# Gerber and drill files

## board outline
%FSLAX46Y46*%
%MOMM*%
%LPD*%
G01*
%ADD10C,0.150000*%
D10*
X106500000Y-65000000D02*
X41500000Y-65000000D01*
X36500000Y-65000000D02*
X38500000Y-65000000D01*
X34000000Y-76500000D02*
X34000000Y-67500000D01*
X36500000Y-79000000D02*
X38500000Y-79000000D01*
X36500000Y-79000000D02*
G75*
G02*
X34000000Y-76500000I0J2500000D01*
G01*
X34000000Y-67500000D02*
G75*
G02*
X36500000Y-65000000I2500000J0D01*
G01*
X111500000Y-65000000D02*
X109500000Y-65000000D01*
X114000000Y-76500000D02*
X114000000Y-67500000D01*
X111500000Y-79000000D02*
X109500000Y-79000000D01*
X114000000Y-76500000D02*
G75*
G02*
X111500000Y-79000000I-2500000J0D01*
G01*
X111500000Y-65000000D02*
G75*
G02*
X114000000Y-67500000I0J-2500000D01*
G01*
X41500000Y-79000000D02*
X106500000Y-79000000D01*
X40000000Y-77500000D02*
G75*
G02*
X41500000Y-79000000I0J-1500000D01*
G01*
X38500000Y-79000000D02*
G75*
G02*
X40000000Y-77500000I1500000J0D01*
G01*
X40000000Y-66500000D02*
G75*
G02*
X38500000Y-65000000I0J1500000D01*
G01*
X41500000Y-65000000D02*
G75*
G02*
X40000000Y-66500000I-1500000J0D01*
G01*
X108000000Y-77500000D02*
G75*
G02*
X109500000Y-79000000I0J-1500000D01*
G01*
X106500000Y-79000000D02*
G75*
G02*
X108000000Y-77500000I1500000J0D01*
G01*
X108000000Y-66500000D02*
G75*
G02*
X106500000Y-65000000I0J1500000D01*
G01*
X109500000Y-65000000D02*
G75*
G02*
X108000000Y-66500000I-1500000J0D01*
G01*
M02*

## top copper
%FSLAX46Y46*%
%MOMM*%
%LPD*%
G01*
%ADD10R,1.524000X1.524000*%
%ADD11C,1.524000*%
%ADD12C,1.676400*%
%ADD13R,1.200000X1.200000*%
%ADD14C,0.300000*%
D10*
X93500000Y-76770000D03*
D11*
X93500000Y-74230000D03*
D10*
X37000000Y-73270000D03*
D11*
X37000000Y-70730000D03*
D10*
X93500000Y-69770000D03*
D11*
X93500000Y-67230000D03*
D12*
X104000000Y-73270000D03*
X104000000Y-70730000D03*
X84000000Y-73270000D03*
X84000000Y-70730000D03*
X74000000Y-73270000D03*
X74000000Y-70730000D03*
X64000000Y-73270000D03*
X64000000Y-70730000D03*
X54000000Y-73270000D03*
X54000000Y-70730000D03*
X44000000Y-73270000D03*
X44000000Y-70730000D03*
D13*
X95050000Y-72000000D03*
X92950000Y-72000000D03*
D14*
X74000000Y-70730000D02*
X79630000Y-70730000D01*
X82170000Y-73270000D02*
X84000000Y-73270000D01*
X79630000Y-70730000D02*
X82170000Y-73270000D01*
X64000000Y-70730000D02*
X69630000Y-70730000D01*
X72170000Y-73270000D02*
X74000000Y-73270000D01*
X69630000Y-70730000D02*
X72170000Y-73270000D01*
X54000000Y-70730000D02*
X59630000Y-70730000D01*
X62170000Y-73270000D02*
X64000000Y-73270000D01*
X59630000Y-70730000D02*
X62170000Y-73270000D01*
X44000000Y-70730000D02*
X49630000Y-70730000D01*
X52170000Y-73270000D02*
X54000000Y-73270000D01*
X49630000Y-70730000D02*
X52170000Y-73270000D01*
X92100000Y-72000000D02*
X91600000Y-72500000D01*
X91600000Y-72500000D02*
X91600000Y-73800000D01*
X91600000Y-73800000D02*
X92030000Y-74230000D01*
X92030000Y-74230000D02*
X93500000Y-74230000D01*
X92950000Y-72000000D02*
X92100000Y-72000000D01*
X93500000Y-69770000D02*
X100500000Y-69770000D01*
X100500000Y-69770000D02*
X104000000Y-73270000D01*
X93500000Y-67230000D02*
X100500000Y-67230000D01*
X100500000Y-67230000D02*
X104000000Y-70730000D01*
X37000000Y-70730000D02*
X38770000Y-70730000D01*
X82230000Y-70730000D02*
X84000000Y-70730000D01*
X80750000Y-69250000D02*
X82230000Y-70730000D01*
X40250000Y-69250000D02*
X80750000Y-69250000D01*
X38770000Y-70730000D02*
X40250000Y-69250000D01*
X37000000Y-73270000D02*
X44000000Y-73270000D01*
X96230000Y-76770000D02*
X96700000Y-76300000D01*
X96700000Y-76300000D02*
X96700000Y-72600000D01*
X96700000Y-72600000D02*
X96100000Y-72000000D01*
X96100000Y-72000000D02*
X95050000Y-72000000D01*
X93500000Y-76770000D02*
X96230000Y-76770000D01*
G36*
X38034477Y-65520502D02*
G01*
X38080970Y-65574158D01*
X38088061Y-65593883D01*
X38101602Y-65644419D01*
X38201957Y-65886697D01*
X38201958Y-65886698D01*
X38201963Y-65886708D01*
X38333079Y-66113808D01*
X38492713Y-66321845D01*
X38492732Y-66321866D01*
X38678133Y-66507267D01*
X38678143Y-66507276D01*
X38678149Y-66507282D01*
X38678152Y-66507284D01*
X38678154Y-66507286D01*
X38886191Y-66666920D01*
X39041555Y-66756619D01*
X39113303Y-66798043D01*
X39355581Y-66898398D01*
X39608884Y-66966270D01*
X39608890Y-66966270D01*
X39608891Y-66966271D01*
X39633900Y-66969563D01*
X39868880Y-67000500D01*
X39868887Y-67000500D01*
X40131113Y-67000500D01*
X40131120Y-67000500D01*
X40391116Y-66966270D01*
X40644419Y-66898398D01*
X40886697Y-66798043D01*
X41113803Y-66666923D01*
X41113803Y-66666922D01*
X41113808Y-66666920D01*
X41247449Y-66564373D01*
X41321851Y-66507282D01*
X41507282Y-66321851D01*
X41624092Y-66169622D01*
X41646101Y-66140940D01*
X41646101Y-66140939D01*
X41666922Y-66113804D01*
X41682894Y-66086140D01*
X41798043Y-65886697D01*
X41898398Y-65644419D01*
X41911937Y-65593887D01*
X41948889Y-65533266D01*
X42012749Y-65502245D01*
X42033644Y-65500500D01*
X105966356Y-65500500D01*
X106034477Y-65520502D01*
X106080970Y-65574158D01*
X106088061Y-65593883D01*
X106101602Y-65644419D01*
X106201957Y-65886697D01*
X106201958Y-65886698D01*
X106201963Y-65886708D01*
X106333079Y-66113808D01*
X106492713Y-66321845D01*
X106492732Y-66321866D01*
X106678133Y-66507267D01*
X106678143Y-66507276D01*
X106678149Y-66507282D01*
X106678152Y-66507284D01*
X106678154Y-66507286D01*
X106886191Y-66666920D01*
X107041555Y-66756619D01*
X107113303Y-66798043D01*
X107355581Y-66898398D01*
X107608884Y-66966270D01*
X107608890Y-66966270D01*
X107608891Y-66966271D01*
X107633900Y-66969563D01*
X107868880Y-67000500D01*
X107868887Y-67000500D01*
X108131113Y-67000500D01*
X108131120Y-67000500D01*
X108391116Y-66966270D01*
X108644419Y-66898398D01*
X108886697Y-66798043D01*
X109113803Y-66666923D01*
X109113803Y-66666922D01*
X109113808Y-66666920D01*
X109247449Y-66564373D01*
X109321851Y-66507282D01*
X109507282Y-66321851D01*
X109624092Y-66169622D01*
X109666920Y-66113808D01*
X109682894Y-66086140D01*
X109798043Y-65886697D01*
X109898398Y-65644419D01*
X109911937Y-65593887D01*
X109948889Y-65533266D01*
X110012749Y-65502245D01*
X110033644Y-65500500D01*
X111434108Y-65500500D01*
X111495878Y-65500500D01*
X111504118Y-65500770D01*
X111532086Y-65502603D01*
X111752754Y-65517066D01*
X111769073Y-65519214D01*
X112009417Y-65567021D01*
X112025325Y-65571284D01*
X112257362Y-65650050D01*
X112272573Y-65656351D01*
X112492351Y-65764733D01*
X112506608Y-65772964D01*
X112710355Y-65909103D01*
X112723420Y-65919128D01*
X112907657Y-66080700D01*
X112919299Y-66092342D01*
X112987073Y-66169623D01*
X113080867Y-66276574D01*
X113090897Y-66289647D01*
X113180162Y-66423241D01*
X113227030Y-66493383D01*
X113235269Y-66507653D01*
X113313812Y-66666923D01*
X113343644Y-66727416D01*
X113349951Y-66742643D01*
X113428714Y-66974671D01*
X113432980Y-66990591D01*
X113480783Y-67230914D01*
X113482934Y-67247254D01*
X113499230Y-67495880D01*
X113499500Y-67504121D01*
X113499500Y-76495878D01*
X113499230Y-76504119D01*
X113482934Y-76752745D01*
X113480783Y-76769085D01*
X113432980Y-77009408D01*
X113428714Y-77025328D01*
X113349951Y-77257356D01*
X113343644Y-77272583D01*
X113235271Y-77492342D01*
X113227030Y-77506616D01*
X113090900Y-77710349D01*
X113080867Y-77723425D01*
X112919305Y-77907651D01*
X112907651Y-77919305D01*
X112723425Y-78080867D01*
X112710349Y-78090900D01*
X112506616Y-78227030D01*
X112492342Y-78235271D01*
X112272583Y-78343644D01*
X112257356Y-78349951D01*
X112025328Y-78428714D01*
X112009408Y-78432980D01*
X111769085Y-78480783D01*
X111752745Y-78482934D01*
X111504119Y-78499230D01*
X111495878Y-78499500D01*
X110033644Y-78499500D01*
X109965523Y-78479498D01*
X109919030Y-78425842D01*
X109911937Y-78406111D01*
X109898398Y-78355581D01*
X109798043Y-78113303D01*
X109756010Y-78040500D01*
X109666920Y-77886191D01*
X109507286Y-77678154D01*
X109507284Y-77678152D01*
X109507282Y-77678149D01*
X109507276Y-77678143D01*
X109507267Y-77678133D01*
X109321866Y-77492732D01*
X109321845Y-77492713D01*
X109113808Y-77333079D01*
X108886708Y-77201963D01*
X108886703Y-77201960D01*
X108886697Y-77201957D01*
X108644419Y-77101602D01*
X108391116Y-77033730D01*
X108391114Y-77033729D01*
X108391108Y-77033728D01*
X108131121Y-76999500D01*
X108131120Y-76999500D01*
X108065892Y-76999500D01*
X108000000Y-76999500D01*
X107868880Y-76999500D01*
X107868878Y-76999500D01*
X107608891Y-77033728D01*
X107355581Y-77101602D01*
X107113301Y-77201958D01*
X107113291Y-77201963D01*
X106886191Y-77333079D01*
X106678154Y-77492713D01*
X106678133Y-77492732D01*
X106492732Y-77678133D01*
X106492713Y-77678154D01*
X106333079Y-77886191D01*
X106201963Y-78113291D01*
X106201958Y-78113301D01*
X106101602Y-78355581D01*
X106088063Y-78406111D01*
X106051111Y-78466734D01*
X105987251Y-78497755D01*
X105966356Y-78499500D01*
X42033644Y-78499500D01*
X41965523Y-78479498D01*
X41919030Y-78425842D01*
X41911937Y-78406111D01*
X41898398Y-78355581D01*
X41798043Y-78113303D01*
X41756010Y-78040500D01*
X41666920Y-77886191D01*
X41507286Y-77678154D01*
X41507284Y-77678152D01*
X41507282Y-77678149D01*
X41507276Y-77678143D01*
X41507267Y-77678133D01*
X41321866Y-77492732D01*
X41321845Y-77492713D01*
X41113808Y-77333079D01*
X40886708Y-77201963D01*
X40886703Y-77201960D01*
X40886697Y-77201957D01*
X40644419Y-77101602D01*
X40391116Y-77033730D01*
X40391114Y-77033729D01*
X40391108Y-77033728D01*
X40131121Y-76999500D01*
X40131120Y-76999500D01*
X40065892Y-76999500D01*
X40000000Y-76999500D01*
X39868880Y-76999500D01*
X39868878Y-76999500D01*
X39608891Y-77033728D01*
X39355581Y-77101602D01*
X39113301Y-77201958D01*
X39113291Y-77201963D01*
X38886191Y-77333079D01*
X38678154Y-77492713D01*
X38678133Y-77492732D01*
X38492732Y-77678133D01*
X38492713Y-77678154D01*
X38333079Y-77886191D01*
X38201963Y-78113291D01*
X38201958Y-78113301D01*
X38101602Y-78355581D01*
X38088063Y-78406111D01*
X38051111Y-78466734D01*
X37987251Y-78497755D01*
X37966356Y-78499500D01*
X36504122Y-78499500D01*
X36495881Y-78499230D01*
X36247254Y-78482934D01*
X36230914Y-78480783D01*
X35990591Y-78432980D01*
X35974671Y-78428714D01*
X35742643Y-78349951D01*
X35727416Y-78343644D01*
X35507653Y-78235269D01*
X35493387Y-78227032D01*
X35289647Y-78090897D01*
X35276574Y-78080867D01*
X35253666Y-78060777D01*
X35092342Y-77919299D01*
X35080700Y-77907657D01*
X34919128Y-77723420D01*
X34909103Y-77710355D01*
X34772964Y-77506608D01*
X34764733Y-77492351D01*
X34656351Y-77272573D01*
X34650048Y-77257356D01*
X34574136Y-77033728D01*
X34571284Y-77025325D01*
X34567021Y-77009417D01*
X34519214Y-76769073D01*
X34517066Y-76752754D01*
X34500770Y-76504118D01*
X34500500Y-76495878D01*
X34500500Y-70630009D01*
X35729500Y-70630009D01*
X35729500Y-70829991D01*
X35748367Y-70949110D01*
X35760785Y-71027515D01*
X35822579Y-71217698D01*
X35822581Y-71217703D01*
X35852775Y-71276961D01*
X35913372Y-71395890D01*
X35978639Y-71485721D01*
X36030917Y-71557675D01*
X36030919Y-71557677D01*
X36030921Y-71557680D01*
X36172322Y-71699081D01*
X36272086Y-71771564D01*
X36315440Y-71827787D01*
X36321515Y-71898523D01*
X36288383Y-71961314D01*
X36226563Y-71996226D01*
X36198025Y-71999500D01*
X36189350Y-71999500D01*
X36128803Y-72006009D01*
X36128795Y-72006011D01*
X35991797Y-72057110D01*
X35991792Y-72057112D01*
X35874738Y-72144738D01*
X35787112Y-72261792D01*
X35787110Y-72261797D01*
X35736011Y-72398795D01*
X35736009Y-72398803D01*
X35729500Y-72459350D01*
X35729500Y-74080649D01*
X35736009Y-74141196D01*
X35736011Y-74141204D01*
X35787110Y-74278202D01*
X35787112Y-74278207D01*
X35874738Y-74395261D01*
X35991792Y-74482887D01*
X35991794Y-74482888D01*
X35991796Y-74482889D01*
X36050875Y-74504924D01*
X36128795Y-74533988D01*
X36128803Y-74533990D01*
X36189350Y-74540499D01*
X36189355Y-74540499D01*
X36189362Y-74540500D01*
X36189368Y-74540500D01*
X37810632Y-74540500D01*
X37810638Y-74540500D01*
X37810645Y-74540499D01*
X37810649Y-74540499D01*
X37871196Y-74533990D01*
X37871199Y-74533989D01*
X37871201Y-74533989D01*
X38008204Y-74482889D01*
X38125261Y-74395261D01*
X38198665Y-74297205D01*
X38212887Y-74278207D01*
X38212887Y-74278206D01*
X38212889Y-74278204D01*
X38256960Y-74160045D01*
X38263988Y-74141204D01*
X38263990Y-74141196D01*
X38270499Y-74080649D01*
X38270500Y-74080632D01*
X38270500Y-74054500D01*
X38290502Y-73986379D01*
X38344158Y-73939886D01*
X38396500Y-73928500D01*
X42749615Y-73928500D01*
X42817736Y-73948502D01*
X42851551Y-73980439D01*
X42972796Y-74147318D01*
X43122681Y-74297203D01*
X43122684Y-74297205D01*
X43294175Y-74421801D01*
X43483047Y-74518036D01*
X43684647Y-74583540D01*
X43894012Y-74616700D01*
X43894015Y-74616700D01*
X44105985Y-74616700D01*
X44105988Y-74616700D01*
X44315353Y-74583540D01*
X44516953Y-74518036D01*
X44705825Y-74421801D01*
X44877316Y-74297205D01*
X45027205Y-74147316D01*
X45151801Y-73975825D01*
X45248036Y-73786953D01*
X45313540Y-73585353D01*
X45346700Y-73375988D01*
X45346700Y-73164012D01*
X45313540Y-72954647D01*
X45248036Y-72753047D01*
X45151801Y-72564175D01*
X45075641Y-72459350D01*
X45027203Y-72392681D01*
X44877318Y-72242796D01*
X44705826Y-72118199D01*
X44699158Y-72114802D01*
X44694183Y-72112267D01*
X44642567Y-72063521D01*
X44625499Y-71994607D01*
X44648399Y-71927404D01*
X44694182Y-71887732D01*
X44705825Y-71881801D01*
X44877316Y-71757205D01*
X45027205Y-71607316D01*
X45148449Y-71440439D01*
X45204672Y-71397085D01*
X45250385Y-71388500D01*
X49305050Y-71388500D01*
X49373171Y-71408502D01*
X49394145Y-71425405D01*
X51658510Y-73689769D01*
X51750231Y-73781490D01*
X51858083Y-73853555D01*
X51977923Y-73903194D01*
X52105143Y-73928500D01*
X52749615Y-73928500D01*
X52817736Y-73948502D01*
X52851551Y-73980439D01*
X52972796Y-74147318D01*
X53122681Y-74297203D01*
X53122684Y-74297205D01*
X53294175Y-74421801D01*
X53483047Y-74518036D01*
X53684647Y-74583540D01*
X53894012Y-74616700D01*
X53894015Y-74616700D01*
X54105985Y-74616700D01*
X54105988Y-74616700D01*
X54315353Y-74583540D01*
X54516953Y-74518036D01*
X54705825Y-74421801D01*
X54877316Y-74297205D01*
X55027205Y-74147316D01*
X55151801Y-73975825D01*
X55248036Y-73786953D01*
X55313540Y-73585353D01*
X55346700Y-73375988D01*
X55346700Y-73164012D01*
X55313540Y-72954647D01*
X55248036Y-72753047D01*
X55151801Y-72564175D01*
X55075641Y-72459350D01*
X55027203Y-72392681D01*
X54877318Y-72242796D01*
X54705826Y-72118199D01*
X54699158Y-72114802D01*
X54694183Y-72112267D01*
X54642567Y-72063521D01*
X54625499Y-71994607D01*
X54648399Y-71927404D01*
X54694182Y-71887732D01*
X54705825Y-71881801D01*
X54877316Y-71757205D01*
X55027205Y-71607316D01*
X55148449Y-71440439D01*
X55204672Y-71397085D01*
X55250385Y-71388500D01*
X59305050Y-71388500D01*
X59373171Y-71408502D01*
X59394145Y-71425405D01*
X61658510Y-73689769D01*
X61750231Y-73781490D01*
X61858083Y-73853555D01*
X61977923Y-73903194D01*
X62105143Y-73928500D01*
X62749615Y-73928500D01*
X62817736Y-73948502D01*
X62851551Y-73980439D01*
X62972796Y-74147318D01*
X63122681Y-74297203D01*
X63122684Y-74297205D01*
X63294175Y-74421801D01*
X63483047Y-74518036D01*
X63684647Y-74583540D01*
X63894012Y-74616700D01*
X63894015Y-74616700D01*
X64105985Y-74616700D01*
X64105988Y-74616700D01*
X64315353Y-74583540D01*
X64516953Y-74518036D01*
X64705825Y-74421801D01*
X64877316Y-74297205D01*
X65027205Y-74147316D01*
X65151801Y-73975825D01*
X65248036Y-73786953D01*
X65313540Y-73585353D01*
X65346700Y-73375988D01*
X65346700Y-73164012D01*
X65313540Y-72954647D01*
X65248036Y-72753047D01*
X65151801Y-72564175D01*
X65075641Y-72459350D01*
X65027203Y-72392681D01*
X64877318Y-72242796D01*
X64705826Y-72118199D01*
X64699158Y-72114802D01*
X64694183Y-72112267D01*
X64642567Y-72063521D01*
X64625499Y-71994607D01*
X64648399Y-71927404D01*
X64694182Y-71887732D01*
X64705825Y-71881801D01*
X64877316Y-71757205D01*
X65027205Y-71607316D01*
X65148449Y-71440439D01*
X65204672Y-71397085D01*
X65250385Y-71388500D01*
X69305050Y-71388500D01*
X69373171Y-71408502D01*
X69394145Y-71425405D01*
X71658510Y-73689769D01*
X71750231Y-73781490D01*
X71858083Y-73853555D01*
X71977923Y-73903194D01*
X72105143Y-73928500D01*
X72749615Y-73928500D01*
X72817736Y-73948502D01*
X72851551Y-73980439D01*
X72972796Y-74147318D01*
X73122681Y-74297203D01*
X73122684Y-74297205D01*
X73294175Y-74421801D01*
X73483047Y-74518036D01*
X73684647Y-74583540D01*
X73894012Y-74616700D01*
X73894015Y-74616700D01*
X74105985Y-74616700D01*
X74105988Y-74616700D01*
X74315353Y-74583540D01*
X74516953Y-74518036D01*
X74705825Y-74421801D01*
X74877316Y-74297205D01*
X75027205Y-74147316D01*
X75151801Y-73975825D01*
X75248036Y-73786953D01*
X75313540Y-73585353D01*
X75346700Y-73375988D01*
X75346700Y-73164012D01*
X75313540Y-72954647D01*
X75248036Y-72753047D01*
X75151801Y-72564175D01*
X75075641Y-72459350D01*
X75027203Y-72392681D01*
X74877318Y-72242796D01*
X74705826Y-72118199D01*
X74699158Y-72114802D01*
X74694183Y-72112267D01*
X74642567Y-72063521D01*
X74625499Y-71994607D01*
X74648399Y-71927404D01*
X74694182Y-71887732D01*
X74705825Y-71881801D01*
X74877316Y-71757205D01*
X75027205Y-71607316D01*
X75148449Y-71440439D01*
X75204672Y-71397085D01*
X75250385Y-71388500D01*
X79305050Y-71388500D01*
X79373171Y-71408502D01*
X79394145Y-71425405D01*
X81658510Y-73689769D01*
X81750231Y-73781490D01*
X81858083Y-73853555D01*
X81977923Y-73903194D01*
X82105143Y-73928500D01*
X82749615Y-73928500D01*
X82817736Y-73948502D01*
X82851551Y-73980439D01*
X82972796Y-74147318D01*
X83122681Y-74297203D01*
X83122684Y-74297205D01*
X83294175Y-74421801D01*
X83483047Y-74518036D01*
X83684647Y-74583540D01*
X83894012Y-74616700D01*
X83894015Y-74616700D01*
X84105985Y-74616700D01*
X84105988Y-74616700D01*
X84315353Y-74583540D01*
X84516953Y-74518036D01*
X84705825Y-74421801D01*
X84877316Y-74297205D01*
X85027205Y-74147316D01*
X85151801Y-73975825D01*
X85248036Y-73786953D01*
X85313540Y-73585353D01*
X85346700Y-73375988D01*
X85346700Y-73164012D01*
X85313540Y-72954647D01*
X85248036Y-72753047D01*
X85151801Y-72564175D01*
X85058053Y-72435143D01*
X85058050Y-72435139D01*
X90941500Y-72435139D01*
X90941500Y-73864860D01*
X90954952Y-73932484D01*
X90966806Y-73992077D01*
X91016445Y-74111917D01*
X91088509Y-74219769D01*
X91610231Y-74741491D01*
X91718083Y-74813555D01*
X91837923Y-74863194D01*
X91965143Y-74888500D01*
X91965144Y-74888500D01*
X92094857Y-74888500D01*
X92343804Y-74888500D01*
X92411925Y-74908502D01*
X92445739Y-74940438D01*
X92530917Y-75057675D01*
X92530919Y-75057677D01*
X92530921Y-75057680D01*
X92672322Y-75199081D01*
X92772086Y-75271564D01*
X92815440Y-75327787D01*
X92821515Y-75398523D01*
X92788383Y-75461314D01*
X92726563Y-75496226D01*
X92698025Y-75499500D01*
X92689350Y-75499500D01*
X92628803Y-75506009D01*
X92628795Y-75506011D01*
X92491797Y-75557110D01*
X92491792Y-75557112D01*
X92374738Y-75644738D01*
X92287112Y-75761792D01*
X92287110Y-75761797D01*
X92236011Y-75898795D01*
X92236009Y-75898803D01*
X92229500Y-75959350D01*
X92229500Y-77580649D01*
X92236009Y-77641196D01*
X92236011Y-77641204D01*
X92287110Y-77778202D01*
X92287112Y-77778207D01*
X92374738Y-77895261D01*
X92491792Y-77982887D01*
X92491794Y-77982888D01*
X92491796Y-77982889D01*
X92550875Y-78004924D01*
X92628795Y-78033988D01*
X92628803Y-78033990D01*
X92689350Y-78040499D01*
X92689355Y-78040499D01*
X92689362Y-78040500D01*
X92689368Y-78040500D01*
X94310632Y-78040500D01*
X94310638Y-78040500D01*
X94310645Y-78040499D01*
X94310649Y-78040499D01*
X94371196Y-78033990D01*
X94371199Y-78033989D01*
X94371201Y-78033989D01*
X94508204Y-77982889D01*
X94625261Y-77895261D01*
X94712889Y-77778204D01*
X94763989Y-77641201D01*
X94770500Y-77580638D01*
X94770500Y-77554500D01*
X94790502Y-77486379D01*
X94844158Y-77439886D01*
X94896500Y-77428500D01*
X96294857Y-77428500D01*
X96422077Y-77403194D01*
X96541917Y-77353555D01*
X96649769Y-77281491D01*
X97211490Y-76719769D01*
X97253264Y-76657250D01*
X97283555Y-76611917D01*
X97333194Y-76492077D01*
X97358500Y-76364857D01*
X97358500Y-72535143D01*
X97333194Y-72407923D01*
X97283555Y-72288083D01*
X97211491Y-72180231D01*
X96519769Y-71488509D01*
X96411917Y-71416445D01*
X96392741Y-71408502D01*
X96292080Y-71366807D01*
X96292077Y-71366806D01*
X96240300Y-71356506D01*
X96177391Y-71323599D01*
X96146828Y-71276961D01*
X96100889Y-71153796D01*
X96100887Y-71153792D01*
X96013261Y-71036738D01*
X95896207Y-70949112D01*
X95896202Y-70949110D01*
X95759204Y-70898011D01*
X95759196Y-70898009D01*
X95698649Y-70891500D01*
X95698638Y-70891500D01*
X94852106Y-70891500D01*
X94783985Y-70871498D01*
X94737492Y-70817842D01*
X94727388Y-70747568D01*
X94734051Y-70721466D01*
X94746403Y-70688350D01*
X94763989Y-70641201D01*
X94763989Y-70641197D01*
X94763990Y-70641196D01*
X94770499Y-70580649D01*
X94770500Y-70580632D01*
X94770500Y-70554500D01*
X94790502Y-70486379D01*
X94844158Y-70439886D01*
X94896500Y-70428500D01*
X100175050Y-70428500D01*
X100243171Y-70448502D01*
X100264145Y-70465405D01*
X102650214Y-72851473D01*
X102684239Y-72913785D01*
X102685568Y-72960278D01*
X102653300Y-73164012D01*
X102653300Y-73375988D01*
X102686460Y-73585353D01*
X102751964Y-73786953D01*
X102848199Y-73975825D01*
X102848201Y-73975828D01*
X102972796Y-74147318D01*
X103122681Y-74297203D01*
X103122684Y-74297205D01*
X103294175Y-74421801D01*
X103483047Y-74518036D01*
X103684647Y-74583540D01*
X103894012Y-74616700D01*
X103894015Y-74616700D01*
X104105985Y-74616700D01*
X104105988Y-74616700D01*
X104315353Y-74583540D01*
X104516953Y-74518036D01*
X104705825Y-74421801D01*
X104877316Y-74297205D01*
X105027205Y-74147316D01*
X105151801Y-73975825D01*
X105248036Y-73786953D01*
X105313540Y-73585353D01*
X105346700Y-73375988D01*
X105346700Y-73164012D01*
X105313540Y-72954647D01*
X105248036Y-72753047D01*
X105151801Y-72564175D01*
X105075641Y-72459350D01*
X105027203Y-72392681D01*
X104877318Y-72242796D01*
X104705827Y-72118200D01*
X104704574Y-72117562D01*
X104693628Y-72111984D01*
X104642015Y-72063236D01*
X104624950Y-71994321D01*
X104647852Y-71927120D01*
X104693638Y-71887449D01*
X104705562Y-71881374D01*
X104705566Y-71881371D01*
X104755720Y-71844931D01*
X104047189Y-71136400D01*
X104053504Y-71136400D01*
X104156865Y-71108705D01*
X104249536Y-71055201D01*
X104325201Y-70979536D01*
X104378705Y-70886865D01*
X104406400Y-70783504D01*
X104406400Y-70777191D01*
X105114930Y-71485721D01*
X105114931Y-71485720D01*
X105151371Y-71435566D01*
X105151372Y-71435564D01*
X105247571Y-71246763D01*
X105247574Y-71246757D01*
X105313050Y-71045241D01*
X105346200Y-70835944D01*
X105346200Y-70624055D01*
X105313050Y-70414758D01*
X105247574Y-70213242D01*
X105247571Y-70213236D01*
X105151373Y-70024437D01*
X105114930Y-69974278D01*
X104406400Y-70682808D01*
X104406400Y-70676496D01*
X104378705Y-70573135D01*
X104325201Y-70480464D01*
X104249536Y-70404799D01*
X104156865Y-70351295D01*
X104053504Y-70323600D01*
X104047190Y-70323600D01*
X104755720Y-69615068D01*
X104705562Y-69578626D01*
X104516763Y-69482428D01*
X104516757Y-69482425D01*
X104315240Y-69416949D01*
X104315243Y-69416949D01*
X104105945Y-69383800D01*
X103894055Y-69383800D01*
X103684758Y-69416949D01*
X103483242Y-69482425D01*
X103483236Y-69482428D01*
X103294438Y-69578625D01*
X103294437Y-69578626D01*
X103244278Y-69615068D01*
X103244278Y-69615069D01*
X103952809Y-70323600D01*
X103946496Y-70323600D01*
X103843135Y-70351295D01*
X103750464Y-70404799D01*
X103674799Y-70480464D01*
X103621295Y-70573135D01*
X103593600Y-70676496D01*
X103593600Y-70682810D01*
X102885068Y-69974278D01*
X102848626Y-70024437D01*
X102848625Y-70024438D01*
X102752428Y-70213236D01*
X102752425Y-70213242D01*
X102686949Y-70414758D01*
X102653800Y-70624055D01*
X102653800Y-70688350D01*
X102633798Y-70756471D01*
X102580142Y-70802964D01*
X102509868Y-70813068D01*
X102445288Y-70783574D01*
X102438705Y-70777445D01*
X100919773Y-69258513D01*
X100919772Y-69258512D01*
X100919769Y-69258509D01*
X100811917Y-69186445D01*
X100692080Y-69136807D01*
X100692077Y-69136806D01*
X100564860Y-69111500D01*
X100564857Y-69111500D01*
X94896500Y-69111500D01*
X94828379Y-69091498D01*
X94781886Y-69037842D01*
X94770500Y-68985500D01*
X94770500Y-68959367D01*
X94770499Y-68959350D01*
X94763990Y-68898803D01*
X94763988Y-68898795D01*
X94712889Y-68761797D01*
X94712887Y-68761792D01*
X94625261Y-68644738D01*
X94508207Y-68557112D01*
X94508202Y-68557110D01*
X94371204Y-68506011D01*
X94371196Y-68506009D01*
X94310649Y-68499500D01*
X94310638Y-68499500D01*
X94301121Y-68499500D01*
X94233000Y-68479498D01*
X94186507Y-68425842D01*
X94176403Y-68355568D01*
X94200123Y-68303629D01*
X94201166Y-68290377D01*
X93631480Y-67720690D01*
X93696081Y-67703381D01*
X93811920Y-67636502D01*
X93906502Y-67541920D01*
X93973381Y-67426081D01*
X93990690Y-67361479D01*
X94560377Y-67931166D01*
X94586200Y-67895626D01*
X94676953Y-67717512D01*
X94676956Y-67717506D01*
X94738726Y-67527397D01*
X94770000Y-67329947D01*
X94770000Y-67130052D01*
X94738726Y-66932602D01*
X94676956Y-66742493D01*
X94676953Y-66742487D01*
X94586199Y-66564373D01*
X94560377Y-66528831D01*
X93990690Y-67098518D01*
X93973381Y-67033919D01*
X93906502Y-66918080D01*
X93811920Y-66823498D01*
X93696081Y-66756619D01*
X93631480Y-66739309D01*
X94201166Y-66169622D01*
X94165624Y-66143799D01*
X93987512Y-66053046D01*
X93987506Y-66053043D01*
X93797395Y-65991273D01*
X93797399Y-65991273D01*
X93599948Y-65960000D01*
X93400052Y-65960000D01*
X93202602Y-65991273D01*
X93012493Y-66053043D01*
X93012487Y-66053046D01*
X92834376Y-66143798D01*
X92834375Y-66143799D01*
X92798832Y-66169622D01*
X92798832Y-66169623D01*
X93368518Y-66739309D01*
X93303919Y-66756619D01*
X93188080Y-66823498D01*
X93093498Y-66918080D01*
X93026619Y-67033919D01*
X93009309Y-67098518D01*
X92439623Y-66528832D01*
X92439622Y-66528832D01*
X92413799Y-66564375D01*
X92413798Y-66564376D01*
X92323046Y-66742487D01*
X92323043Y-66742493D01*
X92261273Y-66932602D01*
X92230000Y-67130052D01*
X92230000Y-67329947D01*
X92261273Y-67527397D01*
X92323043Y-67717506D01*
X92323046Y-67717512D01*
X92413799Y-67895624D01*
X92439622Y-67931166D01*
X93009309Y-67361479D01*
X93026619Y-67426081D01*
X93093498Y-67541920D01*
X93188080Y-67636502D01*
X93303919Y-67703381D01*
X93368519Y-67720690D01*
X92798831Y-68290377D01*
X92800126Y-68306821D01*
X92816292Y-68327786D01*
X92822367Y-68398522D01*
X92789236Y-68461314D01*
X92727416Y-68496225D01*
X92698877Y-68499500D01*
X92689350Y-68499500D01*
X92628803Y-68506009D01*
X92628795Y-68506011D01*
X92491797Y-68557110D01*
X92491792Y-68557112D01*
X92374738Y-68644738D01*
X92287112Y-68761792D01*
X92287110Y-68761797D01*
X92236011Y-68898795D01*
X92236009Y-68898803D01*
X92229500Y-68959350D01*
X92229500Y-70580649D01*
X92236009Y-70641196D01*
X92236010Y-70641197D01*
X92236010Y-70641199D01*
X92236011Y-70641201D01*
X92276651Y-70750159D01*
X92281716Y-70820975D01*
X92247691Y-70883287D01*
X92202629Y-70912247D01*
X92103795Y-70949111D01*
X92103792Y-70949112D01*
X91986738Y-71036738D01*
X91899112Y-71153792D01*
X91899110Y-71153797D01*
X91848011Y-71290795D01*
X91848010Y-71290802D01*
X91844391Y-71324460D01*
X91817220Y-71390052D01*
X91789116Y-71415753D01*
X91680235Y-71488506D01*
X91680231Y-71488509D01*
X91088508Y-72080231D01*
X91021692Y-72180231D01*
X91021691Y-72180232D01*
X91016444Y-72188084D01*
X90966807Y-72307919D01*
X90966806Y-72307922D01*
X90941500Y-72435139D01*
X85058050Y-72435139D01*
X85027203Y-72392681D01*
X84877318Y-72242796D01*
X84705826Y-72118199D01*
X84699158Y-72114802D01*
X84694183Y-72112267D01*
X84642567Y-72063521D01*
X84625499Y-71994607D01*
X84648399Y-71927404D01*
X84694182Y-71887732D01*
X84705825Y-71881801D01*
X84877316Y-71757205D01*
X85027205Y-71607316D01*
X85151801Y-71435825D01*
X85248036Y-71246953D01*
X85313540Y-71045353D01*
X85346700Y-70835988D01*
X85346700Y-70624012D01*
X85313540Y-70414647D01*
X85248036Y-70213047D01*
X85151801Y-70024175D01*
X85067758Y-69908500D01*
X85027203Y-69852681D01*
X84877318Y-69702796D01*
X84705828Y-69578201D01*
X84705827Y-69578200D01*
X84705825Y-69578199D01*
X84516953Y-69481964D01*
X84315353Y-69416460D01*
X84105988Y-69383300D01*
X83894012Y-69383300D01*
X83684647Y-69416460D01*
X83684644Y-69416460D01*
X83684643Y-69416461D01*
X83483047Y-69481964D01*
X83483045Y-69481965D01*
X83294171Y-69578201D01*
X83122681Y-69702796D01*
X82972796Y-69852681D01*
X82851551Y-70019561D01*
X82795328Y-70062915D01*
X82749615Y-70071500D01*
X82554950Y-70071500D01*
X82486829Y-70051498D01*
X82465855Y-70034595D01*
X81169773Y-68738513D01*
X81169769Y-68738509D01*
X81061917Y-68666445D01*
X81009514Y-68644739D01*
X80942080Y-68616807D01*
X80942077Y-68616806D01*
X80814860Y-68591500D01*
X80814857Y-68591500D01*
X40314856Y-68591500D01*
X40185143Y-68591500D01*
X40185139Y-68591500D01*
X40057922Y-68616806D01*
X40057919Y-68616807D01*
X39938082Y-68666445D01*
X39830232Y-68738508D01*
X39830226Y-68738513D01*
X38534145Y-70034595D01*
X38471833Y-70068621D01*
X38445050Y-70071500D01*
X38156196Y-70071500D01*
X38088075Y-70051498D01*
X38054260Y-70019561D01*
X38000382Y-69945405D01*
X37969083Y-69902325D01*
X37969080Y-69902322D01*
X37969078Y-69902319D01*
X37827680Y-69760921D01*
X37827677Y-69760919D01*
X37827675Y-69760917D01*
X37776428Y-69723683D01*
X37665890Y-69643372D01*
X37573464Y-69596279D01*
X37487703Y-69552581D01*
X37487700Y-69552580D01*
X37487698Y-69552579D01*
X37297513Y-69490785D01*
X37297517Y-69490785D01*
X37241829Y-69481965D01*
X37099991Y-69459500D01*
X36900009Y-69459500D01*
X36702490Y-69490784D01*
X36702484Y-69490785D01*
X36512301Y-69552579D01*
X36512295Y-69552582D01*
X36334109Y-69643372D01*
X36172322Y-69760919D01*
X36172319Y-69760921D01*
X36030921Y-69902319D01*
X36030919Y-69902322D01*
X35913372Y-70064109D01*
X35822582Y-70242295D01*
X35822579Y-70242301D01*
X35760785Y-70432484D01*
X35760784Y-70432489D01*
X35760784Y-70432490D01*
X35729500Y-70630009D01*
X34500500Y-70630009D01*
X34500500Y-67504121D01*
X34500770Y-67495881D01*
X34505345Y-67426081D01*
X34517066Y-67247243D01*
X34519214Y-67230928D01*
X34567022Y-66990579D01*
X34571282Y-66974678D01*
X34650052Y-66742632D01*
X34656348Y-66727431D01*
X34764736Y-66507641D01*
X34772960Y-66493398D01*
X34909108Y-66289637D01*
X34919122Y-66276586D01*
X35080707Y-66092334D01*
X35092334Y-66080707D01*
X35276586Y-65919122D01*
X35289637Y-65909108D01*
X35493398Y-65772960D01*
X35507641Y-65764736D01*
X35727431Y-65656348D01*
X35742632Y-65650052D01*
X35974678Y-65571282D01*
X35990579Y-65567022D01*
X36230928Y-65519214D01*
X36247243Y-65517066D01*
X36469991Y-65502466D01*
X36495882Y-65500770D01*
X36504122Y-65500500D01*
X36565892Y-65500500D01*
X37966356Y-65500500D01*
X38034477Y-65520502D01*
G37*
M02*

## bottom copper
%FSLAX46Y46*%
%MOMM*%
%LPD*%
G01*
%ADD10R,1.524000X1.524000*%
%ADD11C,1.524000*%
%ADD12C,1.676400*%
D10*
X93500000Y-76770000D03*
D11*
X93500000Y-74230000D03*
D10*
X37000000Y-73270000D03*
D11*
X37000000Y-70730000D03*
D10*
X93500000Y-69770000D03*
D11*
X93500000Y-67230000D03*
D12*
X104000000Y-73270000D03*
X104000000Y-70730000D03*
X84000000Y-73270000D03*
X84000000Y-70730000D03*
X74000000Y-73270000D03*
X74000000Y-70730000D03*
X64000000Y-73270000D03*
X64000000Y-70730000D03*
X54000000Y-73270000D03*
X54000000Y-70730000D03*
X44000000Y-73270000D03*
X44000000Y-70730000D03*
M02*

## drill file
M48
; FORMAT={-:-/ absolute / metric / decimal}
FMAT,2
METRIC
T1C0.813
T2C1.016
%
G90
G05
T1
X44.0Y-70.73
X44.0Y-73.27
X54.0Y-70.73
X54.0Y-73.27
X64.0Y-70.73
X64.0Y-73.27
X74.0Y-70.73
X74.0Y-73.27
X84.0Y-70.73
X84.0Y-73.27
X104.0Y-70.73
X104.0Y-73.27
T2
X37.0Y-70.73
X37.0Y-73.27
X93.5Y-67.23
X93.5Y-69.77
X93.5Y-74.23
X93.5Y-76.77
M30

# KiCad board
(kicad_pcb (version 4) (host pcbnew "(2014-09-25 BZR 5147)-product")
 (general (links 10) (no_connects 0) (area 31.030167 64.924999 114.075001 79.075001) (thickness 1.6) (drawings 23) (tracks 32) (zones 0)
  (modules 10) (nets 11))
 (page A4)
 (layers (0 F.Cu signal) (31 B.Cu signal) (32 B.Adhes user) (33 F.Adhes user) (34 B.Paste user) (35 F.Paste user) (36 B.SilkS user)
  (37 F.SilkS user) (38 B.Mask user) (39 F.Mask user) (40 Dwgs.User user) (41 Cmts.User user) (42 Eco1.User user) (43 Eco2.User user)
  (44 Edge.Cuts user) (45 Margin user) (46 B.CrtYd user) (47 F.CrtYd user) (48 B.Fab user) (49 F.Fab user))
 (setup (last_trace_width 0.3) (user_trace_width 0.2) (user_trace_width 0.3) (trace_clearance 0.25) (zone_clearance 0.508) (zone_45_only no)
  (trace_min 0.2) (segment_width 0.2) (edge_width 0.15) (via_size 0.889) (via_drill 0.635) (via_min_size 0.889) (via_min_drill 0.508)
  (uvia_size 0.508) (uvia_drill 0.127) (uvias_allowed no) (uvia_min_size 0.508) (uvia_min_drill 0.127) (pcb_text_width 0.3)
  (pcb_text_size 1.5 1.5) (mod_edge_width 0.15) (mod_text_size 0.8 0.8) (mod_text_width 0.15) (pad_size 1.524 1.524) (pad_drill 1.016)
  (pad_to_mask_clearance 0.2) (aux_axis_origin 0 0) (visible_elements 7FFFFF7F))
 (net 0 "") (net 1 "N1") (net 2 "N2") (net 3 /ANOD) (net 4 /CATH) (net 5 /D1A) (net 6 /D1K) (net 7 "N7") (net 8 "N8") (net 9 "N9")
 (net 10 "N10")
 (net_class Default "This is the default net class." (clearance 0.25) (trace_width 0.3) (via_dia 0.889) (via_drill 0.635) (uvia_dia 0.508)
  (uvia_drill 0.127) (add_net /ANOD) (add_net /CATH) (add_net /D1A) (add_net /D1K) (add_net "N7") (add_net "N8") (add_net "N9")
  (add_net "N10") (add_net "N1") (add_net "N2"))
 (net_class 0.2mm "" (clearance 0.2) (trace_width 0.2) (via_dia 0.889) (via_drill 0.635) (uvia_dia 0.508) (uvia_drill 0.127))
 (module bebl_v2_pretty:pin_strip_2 (layer B.Cu) (at 93.5 75.5 90)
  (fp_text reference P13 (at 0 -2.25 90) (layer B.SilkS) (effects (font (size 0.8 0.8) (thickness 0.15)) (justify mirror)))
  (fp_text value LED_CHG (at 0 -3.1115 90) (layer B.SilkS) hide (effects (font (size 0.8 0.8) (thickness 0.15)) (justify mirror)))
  (pad 1 thru_hole rect (at -1.27 0 90) (size 1.524 1.524) (drill 1.016) (layers *.Cu *.Mask B.SilkS) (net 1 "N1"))
  (pad 2 thru_hole circle (at 1.27 0 90) (size 1.524 1.524) (drill 1.016) (layers *.Cu *.Mask B.SilkS) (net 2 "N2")))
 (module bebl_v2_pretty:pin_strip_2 (layer B.Cu) (at 37 72 90)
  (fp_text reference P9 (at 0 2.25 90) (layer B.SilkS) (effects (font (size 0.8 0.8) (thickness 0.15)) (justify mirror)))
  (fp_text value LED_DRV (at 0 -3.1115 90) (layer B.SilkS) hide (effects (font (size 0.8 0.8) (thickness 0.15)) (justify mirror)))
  (pad 1 thru_hole rect (at -1.27 0 90) (size 1.524 1.524) (drill 1.016) (layers *.Cu *.Mask B.SilkS) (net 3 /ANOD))
  (pad 2 thru_hole circle (at 1.27 0 90) (size 1.524 1.524) (drill 1.016) (layers *.Cu *.Mask B.SilkS) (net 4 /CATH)))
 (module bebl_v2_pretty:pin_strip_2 (layer B.Cu) (at 93.5 68.5 90)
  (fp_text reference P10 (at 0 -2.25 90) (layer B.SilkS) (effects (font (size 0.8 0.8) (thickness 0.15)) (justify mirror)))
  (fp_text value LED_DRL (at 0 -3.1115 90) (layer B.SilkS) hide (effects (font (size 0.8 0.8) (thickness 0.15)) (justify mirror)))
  (pad 1 thru_hole rect (at -1.27 0 90) (size 1.524 1.524) (drill 1.016) (layers *.Cu *.Mask B.SilkS) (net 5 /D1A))
  (pad 2 thru_hole circle (at 1.27 0 90) (size 1.524 1.524) (drill 1.016) (layers *.Cu *.Mask B.SilkS) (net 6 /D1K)))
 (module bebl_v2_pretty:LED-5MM (layer F.Cu) (at 104 72 90)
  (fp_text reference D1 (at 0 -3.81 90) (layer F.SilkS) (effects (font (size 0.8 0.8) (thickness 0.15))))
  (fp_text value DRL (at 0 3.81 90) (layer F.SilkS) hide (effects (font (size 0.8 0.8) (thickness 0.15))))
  (pad 1 thru_hole circle (at -1.27 0 90) (size 1.6764 1.6764) (drill 0.8128) (layers *.Cu *.Mask F.SilkS) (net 5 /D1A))
  (pad 2 thru_hole circle (at 1.27 0 90) (size 1.6764 1.6764) (drill 0.8128) (layers *.Cu *.Mask F.SilkS) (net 6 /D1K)))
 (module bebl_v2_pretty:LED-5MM (layer F.Cu) (at 84 72 90)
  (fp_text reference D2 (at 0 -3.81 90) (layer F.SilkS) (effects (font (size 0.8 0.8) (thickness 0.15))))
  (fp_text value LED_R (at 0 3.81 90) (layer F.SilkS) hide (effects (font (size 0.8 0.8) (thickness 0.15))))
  (pad 1 thru_hole circle (at -1.27 0 90) (size 1.6764 1.6764) (drill 0.8128) (layers *.Cu *.Mask F.SilkS) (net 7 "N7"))
  (pad 2 thru_hole circle (at 1.27 0 90) (size 1.6764 1.6764) (drill 0.8128) (layers *.Cu *.Mask F.SilkS) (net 4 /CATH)))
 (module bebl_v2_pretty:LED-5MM (layer F.Cu) (at 74 72 90)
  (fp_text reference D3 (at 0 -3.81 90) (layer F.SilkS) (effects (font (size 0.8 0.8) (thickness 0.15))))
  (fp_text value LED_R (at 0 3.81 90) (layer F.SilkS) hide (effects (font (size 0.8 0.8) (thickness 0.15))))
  (pad 1 thru_hole circle (at -1.27 0 90) (size 1.6764 1.6764) (drill 0.8128) (layers *.Cu *.Mask F.SilkS) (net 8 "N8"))
  (pad 2 thru_hole circle (at 1.27 0 90) (size 1.6764 1.6764) (drill 0.8128) (layers *.Cu *.Mask F.SilkS) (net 7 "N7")))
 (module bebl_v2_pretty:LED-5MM (layer F.Cu) (at 64 72 90)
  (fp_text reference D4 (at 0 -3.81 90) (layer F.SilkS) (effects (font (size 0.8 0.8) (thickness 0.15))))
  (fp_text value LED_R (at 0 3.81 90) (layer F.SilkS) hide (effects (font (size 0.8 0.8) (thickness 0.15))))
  (pad 1 thru_hole circle (at -1.27 0 90) (size 1.6764 1.6764) (drill 0.8128) (layers *.Cu *.Mask F.SilkS) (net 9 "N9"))
  (pad 2 thru_hole circle (at 1.27 0 90) (size 1.6764 1.6764) (drill 0.8128) (layers *.Cu *.Mask F.SilkS) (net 8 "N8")))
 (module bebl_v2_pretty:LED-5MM (layer F.Cu) (at 54 72 90)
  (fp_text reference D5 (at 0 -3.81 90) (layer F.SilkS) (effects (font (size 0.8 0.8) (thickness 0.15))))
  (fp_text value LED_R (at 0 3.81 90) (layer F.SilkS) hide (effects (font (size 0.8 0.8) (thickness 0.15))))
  (pad 1 thru_hole circle (at -1.27 0 90) (size 1.6764 1.6764) (drill 0.8128) (layers *.Cu *.Mask F.SilkS) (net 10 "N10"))
  (pad 2 thru_hole circle (at 1.27 0 90) (size 1.6764 1.6764) (drill 0.8128) (layers *.Cu *.Mask F.SilkS) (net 9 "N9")))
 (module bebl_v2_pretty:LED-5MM (layer F.Cu) (at 44 72 90)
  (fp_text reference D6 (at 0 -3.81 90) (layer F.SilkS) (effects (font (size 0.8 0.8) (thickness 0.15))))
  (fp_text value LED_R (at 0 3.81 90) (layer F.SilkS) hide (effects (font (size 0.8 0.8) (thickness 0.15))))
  (pad 1 thru_hole circle (at -1.27 0 90) (size 1.6764 1.6764) (drill 0.8128) (layers *.Cu *.Mask F.SilkS) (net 3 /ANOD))
  (pad 2 thru_hole circle (at 1.27 0 90) (size 1.6764 1.6764) (drill 0.8128) (layers *.Cu *.Mask F.SilkS) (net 10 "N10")))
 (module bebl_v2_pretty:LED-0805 (layer F.Cu) (at 94 72 180)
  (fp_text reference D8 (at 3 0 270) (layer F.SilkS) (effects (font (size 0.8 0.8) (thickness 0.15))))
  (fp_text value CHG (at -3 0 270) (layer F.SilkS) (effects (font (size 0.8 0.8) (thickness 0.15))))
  (pad 1 smd rect (at -1.05 0 180) (size 1.2 1.2) (layers F.Cu F.Paste F.Mask) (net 1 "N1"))
  (pad 2 smd rect (at 1.05 0 180) (size 1.2 1.2) (layers F.Cu F.Paste F.Mask) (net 2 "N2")))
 (gr_line (start 106.5 65) (end 41.5 65) (angle 90) (layer Edge.Cuts) (width 0.15))
 (gr_line (start 36.5 65) (end 38.5 65) (angle 90) (layer Edge.Cuts) (width 0.15))
 (gr_line (start 34 76.5) (end 34 67.5) (angle 90) (layer Edge.Cuts) (width 0.15))
 (gr_line (start 36.5 79) (end 38.5 79) (angle 90) (layer Edge.Cuts) (width 0.15))
 (gr_arc (start 36.5 76.5) (end 36.5 79) (angle 90) (layer Edge.Cuts) (width 0.15))
 (gr_arc (start 36.5 67.5) (end 34 67.5) (angle 90) (layer Edge.Cuts) (width 0.15))
 (gr_line (start 111.5 65) (end 109.5 65) (angle 90) (layer Edge.Cuts) (width 0.15))
 (gr_line (start 114 76.5) (end 114 67.5) (angle 90) (layer Edge.Cuts) (width 0.15))
 (gr_line (start 111.5 79) (end 109.5 79) (angle 90) (layer Edge.Cuts) (width 0.15))
 (gr_arc (start 111.5 76.5) (end 114 76.5) (angle 90) (layer Edge.Cuts) (width 0.15))
 (gr_arc (start 111.5 67.5) (end 111.5 65) (angle 90) (layer Edge.Cuts) (width 0.15))
 (gr_line (start 41.5 79) (end 106.5 79) (angle 90) (layer Edge.Cuts) (width 0.15))
 (gr_arc (start 40 79) (end 40 77.5) (angle 90) (layer Edge.Cuts) (width 0.15))
 (gr_arc (start 40 79) (end 38.5 79) (angle 90) (layer Edge.Cuts) (width 0.15))
 (gr_arc (start 40 65) (end 40 66.5) (angle 90) (layer Edge.Cuts) (width 0.15))
 (gr_arc (start 40 65) (end 41.5 65) (angle 90) (layer Edge.Cuts) (width 0.15))
 (gr_arc (start 108 79) (end 108 77.5) (angle 90) (layer Edge.Cuts) (width 0.15))
 (gr_arc (start 108 79) (end 106.5 79) (angle 90) (layer Edge.Cuts) (width 0.15))
 (gr_arc (start 108 65) (end 108 66.5) (angle 90) (layer Edge.Cuts) (width 0.15))
 (gr_arc (start 108 65) (end 109.5 65) (angle 90) (layer Edge.Cuts) (width 0.15))
 (segment (start 74 70.73) (end 79.63 70.73) (width 0.3) (layer F.Cu) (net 7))
 (segment (start 82.17 73.27) (end 84 73.27) (width 0.3) (layer F.Cu) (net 7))
 (segment (start 79.63 70.73) (end 82.17 73.27) (width 0.3) (layer F.Cu) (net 7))
 (segment (start 64 70.73) (end 69.63 70.73) (width 0.3) (layer F.Cu) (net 8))
 (segment (start 72.17 73.27) (end 74 73.27) (width 0.3) (layer F.Cu) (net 8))
 (segment (start 69.63 70.73) (end 72.17 73.27) (width 0.3) (layer F.Cu) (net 8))
 (segment (start 54 70.73) (end 59.63 70.73) (width 0.3) (layer F.Cu) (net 9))
 (segment (start 62.17 73.27) (end 64 73.27) (width 0.3) (layer F.Cu) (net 9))
 (segment (start 59.63 70.73) (end 62.17 73.27) (width 0.3) (layer F.Cu) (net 9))
 (segment (start 44 70.73) (end 49.63 70.73) (width 0.3) (layer F.Cu) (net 10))
 (segment (start 52.17 73.27) (end 54 73.27) (width 0.3) (layer F.Cu) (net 10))
 (segment (start 49.63 70.73) (end 52.17 73.27) (width 0.3) (layer F.Cu) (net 10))
 (segment (start 92.1 72) (end 91.6 72.5) (width 0.3) (layer F.Cu) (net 2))
 (segment (start 91.6 72.5) (end 91.6 73.8) (width 0.3) (layer F.Cu) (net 2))
 (segment (start 91.6 73.8) (end 92.03 74.23) (width 0.3) (layer F.Cu) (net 2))
 (segment (start 92.03 74.23) (end 93.5 74.23) (width 0.3) (layer F.Cu) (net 2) (status 20))
 (segment (start 92.95 72) (end 92.1 72) (width 0.3) (layer F.Cu) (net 2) (status 10))
 (segment (start 93.5 69.77) (end 100.5 69.77) (width 0.3) (layer F.Cu) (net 5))
 (segment (start 100.5 69.77) (end 104 73.27) (width 0.3) (layer F.Cu) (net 5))
 (segment (start 93.5 67.23) (end 100.5 67.23) (width 0.3) (layer F.Cu) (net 6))
 (segment (start 100.5 67.23) (end 104 70.73) (width 0.3) (layer F.Cu) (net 6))
 (segment (start 37 70.73) (end 38.77 70.73) (width 0.3) (layer F.Cu) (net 4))
 (segment (start 82.23 70.73) (end 84 70.73) (width 0.3) (layer F.Cu) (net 4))
 (segment (start 80.75 69.25) (end 82.23 70.73) (width 0.3) (layer F.Cu) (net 4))
 (segment (start 40.25 69.25) (end 80.75 69.25) (width 0.3) (layer F.Cu) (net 4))
 (segment (start 38.77 70.73) (end 40.25 69.25) (width 0.3) (layer F.Cu) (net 4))
 (segment (start 37 73.27) (end 44 73.27) (width 0.3) (layer F.Cu) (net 3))
 (segment (start 96.23 76.77) (end 96.7 76.3) (width 0.3) (layer F.Cu) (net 1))
 (segment (start 96.7 76.3) (end 96.7 72.6) (width 0.3) (layer F.Cu) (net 1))
 (segment (start 96.7 72.6) (end 96.1 72) (width 0.3) (layer F.Cu) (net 1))
 (segment (start 96.1 72) (end 95.05 72) (width 0.3) (layer F.Cu) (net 1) (status 20))
 (segment (start 93.5 76.77) (end 96.23 76.77) (width 0.3) (layer F.Cu) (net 1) (status 10))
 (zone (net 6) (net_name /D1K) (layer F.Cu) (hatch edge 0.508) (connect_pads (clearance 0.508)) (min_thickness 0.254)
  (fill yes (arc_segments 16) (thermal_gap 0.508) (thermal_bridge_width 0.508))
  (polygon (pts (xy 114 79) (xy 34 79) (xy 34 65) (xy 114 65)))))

